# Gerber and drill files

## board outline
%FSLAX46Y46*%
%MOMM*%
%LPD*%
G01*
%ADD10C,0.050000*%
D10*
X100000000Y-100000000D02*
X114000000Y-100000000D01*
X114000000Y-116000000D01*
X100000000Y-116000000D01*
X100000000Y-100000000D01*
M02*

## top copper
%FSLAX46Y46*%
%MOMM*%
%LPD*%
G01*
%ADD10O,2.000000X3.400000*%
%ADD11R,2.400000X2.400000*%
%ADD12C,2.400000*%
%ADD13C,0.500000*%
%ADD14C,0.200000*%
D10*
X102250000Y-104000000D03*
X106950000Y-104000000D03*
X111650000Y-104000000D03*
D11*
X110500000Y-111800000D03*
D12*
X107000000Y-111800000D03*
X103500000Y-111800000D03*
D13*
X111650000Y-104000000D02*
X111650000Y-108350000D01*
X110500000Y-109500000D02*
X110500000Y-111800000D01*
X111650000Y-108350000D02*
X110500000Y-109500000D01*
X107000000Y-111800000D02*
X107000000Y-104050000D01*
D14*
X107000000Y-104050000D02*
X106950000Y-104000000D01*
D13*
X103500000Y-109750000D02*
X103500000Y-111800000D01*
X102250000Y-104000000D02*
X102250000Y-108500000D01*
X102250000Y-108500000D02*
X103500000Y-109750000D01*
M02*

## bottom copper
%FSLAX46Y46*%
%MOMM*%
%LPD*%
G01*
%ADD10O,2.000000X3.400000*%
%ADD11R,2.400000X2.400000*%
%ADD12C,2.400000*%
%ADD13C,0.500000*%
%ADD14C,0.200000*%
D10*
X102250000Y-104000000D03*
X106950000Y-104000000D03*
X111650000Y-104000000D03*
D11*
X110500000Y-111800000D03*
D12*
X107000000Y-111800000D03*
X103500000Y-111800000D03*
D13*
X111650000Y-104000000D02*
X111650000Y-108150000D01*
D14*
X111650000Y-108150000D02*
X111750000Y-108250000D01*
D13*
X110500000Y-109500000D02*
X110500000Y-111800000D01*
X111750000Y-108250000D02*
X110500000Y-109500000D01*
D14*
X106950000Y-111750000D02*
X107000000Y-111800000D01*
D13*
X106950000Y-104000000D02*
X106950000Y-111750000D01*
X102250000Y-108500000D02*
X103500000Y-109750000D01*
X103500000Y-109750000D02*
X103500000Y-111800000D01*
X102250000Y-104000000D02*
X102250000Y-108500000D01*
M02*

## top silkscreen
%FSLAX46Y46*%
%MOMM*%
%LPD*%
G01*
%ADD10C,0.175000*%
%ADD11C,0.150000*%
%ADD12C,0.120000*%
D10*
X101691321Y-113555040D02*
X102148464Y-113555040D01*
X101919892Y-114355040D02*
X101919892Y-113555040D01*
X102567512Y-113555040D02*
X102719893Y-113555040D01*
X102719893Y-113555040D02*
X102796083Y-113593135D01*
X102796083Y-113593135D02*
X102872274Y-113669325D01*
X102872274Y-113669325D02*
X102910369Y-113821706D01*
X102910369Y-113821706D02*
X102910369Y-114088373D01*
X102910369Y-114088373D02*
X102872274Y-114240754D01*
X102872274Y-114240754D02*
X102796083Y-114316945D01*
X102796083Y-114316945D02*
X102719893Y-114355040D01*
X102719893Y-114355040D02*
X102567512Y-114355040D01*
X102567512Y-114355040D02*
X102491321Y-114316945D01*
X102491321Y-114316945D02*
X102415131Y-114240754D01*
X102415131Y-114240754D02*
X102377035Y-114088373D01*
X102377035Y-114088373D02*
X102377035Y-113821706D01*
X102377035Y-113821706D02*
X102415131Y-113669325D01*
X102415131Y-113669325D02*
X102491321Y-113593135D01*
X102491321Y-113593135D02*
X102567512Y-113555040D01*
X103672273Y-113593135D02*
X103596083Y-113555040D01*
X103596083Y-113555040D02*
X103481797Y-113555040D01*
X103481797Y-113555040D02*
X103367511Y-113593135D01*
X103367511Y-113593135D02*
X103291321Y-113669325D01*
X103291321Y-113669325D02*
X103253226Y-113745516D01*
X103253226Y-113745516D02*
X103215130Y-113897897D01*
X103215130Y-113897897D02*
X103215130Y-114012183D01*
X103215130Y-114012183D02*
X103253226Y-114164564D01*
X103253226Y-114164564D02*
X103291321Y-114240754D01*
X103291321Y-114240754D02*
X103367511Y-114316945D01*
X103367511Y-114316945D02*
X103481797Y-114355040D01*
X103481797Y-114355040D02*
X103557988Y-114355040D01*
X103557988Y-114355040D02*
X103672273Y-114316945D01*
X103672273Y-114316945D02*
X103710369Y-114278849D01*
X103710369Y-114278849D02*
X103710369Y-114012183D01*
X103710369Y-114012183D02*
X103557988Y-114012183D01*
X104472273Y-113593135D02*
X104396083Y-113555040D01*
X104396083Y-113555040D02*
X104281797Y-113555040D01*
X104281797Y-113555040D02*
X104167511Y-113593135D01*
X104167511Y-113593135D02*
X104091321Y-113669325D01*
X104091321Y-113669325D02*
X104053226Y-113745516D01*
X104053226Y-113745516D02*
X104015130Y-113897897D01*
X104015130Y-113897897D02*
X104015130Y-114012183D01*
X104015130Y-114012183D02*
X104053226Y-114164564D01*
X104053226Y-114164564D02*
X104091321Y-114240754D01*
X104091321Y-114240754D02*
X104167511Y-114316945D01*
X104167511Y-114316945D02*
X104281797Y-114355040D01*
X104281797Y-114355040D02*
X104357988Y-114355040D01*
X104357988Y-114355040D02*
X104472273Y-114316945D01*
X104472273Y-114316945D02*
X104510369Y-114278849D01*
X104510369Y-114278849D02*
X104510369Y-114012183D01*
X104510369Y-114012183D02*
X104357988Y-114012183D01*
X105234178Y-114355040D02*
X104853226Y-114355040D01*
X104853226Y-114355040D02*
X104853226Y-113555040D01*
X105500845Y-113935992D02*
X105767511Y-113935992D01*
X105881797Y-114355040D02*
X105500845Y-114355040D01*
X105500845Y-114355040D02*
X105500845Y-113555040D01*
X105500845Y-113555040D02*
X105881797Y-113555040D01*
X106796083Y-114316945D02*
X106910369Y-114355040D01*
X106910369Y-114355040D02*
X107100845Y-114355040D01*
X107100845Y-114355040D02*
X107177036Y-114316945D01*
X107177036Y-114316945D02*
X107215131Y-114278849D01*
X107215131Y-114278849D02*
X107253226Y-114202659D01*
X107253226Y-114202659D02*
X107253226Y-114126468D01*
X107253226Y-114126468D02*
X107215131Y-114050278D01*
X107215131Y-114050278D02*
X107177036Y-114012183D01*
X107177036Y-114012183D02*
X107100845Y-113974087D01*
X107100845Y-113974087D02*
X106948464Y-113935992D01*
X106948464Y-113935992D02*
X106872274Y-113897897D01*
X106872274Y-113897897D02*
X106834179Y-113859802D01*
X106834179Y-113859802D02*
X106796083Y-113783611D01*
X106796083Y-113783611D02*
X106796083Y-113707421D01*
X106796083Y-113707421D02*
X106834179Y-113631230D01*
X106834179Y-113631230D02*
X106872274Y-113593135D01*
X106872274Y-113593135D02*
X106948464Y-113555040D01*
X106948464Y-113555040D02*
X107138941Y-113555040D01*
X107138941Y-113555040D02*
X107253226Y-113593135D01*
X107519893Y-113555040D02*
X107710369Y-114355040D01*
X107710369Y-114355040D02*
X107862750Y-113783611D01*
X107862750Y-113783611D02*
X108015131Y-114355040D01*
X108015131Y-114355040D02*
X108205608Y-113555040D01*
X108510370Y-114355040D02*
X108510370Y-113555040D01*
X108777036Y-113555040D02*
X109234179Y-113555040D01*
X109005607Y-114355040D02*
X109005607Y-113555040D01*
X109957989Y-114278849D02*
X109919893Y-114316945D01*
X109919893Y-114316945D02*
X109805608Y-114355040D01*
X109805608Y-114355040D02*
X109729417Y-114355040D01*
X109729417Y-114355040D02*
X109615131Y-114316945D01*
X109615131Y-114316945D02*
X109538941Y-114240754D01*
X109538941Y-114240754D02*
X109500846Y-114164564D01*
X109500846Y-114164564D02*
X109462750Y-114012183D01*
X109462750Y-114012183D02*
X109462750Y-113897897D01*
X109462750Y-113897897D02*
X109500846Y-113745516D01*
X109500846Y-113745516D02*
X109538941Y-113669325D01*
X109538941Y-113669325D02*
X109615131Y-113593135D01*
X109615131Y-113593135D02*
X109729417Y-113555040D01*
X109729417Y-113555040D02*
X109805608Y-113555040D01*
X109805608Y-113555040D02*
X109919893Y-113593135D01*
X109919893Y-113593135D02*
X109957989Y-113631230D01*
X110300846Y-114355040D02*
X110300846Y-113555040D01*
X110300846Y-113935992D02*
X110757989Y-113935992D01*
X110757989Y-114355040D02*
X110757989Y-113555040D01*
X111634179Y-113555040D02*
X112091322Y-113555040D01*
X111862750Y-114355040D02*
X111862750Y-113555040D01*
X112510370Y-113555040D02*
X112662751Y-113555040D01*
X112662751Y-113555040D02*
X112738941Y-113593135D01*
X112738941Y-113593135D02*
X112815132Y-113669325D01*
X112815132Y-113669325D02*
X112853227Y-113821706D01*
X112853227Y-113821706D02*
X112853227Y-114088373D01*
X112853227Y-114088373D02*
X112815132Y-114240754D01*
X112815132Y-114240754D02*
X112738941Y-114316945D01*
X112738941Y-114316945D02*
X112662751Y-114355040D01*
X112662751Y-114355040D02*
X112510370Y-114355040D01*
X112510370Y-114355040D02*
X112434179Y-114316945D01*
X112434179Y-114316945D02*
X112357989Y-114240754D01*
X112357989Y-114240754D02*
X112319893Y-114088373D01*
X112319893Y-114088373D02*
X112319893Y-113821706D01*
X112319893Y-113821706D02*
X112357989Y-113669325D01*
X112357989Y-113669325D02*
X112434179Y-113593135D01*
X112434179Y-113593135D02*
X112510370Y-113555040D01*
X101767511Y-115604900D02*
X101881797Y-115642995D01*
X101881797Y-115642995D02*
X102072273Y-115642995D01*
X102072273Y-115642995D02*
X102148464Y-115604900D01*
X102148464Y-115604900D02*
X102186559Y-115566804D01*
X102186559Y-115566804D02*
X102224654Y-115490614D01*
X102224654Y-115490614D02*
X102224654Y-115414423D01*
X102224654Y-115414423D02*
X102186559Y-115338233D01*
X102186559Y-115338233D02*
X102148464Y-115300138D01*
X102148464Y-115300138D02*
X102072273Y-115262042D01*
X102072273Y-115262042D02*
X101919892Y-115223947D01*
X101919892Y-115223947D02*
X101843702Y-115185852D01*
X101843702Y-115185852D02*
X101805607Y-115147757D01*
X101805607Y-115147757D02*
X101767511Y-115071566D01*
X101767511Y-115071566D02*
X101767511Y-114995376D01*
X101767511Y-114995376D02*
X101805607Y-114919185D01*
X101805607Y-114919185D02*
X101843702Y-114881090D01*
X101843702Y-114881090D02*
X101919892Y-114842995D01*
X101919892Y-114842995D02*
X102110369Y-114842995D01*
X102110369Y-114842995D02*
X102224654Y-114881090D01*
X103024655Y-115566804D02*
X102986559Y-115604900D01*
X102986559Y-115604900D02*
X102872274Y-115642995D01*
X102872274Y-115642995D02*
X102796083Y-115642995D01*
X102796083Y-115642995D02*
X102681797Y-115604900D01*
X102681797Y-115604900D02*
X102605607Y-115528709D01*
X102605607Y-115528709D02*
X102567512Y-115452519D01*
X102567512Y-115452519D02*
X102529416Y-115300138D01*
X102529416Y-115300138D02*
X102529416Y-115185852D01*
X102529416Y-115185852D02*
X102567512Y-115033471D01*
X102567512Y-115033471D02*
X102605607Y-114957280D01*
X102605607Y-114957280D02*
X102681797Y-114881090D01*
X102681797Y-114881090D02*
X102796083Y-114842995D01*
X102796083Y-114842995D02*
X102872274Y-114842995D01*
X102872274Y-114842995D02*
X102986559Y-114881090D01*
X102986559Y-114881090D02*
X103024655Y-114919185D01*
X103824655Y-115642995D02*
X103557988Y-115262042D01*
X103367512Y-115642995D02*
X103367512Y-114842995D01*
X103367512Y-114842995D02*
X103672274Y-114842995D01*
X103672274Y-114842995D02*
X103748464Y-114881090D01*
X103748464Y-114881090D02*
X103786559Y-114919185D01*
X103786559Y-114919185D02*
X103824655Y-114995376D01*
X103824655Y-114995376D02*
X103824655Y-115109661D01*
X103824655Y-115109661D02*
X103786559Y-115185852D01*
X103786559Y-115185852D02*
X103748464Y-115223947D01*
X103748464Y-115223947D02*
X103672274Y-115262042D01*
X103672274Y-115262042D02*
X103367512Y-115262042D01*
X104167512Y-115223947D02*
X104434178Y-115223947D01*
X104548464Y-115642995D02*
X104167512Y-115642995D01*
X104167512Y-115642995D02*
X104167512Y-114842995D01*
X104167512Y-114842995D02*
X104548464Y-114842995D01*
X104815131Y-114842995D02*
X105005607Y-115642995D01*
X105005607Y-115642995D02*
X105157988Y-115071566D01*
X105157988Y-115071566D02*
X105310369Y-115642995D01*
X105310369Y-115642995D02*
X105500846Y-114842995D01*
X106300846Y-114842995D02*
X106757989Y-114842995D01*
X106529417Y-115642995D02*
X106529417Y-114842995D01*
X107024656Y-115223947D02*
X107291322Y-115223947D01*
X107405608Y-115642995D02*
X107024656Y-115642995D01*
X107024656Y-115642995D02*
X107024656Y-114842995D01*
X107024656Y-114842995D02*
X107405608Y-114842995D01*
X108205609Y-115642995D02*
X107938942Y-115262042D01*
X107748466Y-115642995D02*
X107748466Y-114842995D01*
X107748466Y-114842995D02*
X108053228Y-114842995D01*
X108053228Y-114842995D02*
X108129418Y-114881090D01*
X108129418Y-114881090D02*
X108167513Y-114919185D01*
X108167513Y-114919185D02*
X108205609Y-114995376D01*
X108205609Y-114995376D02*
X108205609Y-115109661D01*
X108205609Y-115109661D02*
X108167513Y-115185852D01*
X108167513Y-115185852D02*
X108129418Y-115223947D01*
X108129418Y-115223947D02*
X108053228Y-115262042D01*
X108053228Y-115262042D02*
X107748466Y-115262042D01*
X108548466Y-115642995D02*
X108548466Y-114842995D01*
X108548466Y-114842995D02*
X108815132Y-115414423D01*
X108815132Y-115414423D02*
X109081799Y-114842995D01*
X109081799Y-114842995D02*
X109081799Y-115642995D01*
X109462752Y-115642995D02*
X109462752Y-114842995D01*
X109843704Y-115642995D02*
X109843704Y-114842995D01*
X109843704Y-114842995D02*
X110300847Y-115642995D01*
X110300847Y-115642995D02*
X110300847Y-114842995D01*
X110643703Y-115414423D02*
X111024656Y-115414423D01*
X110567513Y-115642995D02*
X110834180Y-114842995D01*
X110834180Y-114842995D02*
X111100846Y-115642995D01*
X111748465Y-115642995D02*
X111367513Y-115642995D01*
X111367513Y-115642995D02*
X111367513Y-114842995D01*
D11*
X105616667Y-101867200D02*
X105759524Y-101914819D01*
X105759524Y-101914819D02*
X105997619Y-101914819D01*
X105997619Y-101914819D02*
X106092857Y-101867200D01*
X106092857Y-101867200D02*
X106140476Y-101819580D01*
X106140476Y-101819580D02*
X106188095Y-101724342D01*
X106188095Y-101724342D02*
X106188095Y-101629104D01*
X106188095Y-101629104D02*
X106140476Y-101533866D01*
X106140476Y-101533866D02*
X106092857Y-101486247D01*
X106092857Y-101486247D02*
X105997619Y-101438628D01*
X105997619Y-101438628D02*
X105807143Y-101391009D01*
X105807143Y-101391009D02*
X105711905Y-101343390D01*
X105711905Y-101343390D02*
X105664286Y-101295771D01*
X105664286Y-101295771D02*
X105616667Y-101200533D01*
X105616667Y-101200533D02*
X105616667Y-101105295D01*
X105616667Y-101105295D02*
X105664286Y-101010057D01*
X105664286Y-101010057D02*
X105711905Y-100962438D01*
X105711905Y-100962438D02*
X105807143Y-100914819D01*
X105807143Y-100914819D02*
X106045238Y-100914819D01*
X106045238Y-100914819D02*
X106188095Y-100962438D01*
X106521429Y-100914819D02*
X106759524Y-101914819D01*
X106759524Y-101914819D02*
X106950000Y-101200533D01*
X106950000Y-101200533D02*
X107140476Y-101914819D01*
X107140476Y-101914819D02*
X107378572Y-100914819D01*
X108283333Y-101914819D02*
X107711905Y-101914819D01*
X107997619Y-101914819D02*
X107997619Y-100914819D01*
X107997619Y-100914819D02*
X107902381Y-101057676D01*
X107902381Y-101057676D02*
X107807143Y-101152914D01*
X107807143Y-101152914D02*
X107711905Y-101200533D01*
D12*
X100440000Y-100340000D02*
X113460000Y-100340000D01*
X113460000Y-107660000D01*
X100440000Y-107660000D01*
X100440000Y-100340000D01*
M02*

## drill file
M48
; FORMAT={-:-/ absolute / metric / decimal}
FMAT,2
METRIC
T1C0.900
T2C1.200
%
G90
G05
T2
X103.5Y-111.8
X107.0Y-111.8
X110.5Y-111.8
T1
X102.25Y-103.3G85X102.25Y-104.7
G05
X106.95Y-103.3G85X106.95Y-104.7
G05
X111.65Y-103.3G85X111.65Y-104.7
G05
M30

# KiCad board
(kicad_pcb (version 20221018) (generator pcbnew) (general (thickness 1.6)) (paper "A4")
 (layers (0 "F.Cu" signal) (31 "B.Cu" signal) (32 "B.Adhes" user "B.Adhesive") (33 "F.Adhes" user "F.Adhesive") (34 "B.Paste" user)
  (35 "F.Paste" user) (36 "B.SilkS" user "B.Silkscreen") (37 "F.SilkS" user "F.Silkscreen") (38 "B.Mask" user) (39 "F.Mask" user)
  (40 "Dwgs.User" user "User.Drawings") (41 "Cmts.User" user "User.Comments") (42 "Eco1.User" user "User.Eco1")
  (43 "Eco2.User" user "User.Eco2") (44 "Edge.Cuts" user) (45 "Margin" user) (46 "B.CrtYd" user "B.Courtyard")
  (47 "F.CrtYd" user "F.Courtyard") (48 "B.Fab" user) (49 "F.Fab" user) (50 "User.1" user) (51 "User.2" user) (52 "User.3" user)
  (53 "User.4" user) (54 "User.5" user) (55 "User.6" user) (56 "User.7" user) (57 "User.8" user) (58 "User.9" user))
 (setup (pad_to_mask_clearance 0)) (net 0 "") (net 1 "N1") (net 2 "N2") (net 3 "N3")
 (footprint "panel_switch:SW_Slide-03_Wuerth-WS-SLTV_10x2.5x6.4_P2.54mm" (layer "F.Cu") (at 106.95 104)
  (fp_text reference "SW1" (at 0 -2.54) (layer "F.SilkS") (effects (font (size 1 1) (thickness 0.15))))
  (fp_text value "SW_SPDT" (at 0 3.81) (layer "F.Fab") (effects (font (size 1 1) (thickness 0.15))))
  (fp_rect (start -6.51 -3.66) (end 6.51 3.66) (stroke (width 0.12) (type default)) (fill none) (layer "F.SilkS"))
  (pad "1" thru_hole oval (at -4.7 0) (size 2 3.4) (drill oval 0.9 2.3) (layers "*.Cu" "*.Mask") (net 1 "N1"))
  (pad "2" thru_hole oval (at 0 0) (size 2 3.4) (drill oval 0.9 2.3) (layers "*.Cu" "*.Mask") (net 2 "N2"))
  (pad "3" thru_hole oval (at 4.7 0) (size 2 3.4) (drill oval 0.9 2.3) (layers "*.Cu" "*.Mask") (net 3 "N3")))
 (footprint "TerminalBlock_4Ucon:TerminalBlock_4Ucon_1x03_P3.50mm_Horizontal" (layer "B.Cu") (at 110.5 111.8 180)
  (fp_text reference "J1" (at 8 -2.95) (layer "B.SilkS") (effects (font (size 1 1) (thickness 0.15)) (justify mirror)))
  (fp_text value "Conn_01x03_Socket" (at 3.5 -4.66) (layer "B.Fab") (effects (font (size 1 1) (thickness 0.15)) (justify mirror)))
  (pad "1" thru_hole rect (at 0 0 180) (size 2.4 2.4) (drill 1.2) (layers "*.Cu" "*.Mask") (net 3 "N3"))
  (pad "2" thru_hole circle (at 3.5 0 180) (size 2.4 2.4) (drill 1.2) (layers "*.Cu" "*.Mask") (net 2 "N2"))
  (pad "3" thru_hole circle (at 7 0 180) (size 2.4 2.4) (drill 1.2) (layers "*.Cu" "*.Mask") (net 1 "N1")))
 (gr_rect (start 100 100) (end 114 116) (stroke (width 0.05) (type default)) (fill none) (layer "Edge.Cuts"))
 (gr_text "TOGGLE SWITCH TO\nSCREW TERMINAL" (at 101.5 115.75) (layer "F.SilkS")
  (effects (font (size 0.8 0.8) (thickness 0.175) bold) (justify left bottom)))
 (segment (start 111.65 104) (end 111.65 108.35) (width 0.5) (layer "F.Cu") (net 3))
 (segment (start 110.5 109.5) (end 110.5 111.8) (width 0.5) (layer "F.Cu") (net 3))
 (segment (start 111.65 108.35) (end 110.5 109.5) (width 0.5) (layer "F.Cu") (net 3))
 (segment (start 111.65 104) (end 111.65 108.15) (width 0.5) (layer "B.Cu") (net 3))
 (segment (start 111.65 108.15) (end 111.75 108.25) (width 0.2) (layer "B.Cu") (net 3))
 (segment (start 110.5 109.5) (end 110.5 111.8) (width 0.5) (layer "B.Cu") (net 3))
 (segment (start 111.75 108.25) (end 110.5 109.5) (width 0.5) (layer "B.Cu") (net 3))
 (segment (start 107 111.8) (end 107 104.05) (width 0.5) (layer "F.Cu") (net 2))
 (segment (start 107 104.05) (end 106.95 104) (width 0.2) (layer "F.Cu") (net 2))
 (segment (start 106.95 111.75) (end 107 111.8) (width 0.2) (layer "B.Cu") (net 2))
 (segment (start 106.95 104) (end 106.95 111.75) (width 0.5) (layer "B.Cu") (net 2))
 (segment (start 103.5 109.75) (end 103.5 111.8) (width 0.5) (layer "F.Cu") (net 1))
 (segment (start 102.25 104) (end 102.25 108.5) (width 0.5) (layer "F.Cu") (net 1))
 (segment (start 102.25 108.5) (end 103.5 109.75) (width 0.5) (layer "F.Cu") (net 1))
 (segment (start 102.25 108.5) (end 103.5 109.75) (width 0.5) (layer "B.Cu") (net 1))
 (segment (start 103.5 109.75) (end 103.5 111.8) (width 0.5) (layer "B.Cu") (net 1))
 (segment (start 102.25 104) (end 102.25 108.5) (width 0.5) (layer "B.Cu") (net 1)))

